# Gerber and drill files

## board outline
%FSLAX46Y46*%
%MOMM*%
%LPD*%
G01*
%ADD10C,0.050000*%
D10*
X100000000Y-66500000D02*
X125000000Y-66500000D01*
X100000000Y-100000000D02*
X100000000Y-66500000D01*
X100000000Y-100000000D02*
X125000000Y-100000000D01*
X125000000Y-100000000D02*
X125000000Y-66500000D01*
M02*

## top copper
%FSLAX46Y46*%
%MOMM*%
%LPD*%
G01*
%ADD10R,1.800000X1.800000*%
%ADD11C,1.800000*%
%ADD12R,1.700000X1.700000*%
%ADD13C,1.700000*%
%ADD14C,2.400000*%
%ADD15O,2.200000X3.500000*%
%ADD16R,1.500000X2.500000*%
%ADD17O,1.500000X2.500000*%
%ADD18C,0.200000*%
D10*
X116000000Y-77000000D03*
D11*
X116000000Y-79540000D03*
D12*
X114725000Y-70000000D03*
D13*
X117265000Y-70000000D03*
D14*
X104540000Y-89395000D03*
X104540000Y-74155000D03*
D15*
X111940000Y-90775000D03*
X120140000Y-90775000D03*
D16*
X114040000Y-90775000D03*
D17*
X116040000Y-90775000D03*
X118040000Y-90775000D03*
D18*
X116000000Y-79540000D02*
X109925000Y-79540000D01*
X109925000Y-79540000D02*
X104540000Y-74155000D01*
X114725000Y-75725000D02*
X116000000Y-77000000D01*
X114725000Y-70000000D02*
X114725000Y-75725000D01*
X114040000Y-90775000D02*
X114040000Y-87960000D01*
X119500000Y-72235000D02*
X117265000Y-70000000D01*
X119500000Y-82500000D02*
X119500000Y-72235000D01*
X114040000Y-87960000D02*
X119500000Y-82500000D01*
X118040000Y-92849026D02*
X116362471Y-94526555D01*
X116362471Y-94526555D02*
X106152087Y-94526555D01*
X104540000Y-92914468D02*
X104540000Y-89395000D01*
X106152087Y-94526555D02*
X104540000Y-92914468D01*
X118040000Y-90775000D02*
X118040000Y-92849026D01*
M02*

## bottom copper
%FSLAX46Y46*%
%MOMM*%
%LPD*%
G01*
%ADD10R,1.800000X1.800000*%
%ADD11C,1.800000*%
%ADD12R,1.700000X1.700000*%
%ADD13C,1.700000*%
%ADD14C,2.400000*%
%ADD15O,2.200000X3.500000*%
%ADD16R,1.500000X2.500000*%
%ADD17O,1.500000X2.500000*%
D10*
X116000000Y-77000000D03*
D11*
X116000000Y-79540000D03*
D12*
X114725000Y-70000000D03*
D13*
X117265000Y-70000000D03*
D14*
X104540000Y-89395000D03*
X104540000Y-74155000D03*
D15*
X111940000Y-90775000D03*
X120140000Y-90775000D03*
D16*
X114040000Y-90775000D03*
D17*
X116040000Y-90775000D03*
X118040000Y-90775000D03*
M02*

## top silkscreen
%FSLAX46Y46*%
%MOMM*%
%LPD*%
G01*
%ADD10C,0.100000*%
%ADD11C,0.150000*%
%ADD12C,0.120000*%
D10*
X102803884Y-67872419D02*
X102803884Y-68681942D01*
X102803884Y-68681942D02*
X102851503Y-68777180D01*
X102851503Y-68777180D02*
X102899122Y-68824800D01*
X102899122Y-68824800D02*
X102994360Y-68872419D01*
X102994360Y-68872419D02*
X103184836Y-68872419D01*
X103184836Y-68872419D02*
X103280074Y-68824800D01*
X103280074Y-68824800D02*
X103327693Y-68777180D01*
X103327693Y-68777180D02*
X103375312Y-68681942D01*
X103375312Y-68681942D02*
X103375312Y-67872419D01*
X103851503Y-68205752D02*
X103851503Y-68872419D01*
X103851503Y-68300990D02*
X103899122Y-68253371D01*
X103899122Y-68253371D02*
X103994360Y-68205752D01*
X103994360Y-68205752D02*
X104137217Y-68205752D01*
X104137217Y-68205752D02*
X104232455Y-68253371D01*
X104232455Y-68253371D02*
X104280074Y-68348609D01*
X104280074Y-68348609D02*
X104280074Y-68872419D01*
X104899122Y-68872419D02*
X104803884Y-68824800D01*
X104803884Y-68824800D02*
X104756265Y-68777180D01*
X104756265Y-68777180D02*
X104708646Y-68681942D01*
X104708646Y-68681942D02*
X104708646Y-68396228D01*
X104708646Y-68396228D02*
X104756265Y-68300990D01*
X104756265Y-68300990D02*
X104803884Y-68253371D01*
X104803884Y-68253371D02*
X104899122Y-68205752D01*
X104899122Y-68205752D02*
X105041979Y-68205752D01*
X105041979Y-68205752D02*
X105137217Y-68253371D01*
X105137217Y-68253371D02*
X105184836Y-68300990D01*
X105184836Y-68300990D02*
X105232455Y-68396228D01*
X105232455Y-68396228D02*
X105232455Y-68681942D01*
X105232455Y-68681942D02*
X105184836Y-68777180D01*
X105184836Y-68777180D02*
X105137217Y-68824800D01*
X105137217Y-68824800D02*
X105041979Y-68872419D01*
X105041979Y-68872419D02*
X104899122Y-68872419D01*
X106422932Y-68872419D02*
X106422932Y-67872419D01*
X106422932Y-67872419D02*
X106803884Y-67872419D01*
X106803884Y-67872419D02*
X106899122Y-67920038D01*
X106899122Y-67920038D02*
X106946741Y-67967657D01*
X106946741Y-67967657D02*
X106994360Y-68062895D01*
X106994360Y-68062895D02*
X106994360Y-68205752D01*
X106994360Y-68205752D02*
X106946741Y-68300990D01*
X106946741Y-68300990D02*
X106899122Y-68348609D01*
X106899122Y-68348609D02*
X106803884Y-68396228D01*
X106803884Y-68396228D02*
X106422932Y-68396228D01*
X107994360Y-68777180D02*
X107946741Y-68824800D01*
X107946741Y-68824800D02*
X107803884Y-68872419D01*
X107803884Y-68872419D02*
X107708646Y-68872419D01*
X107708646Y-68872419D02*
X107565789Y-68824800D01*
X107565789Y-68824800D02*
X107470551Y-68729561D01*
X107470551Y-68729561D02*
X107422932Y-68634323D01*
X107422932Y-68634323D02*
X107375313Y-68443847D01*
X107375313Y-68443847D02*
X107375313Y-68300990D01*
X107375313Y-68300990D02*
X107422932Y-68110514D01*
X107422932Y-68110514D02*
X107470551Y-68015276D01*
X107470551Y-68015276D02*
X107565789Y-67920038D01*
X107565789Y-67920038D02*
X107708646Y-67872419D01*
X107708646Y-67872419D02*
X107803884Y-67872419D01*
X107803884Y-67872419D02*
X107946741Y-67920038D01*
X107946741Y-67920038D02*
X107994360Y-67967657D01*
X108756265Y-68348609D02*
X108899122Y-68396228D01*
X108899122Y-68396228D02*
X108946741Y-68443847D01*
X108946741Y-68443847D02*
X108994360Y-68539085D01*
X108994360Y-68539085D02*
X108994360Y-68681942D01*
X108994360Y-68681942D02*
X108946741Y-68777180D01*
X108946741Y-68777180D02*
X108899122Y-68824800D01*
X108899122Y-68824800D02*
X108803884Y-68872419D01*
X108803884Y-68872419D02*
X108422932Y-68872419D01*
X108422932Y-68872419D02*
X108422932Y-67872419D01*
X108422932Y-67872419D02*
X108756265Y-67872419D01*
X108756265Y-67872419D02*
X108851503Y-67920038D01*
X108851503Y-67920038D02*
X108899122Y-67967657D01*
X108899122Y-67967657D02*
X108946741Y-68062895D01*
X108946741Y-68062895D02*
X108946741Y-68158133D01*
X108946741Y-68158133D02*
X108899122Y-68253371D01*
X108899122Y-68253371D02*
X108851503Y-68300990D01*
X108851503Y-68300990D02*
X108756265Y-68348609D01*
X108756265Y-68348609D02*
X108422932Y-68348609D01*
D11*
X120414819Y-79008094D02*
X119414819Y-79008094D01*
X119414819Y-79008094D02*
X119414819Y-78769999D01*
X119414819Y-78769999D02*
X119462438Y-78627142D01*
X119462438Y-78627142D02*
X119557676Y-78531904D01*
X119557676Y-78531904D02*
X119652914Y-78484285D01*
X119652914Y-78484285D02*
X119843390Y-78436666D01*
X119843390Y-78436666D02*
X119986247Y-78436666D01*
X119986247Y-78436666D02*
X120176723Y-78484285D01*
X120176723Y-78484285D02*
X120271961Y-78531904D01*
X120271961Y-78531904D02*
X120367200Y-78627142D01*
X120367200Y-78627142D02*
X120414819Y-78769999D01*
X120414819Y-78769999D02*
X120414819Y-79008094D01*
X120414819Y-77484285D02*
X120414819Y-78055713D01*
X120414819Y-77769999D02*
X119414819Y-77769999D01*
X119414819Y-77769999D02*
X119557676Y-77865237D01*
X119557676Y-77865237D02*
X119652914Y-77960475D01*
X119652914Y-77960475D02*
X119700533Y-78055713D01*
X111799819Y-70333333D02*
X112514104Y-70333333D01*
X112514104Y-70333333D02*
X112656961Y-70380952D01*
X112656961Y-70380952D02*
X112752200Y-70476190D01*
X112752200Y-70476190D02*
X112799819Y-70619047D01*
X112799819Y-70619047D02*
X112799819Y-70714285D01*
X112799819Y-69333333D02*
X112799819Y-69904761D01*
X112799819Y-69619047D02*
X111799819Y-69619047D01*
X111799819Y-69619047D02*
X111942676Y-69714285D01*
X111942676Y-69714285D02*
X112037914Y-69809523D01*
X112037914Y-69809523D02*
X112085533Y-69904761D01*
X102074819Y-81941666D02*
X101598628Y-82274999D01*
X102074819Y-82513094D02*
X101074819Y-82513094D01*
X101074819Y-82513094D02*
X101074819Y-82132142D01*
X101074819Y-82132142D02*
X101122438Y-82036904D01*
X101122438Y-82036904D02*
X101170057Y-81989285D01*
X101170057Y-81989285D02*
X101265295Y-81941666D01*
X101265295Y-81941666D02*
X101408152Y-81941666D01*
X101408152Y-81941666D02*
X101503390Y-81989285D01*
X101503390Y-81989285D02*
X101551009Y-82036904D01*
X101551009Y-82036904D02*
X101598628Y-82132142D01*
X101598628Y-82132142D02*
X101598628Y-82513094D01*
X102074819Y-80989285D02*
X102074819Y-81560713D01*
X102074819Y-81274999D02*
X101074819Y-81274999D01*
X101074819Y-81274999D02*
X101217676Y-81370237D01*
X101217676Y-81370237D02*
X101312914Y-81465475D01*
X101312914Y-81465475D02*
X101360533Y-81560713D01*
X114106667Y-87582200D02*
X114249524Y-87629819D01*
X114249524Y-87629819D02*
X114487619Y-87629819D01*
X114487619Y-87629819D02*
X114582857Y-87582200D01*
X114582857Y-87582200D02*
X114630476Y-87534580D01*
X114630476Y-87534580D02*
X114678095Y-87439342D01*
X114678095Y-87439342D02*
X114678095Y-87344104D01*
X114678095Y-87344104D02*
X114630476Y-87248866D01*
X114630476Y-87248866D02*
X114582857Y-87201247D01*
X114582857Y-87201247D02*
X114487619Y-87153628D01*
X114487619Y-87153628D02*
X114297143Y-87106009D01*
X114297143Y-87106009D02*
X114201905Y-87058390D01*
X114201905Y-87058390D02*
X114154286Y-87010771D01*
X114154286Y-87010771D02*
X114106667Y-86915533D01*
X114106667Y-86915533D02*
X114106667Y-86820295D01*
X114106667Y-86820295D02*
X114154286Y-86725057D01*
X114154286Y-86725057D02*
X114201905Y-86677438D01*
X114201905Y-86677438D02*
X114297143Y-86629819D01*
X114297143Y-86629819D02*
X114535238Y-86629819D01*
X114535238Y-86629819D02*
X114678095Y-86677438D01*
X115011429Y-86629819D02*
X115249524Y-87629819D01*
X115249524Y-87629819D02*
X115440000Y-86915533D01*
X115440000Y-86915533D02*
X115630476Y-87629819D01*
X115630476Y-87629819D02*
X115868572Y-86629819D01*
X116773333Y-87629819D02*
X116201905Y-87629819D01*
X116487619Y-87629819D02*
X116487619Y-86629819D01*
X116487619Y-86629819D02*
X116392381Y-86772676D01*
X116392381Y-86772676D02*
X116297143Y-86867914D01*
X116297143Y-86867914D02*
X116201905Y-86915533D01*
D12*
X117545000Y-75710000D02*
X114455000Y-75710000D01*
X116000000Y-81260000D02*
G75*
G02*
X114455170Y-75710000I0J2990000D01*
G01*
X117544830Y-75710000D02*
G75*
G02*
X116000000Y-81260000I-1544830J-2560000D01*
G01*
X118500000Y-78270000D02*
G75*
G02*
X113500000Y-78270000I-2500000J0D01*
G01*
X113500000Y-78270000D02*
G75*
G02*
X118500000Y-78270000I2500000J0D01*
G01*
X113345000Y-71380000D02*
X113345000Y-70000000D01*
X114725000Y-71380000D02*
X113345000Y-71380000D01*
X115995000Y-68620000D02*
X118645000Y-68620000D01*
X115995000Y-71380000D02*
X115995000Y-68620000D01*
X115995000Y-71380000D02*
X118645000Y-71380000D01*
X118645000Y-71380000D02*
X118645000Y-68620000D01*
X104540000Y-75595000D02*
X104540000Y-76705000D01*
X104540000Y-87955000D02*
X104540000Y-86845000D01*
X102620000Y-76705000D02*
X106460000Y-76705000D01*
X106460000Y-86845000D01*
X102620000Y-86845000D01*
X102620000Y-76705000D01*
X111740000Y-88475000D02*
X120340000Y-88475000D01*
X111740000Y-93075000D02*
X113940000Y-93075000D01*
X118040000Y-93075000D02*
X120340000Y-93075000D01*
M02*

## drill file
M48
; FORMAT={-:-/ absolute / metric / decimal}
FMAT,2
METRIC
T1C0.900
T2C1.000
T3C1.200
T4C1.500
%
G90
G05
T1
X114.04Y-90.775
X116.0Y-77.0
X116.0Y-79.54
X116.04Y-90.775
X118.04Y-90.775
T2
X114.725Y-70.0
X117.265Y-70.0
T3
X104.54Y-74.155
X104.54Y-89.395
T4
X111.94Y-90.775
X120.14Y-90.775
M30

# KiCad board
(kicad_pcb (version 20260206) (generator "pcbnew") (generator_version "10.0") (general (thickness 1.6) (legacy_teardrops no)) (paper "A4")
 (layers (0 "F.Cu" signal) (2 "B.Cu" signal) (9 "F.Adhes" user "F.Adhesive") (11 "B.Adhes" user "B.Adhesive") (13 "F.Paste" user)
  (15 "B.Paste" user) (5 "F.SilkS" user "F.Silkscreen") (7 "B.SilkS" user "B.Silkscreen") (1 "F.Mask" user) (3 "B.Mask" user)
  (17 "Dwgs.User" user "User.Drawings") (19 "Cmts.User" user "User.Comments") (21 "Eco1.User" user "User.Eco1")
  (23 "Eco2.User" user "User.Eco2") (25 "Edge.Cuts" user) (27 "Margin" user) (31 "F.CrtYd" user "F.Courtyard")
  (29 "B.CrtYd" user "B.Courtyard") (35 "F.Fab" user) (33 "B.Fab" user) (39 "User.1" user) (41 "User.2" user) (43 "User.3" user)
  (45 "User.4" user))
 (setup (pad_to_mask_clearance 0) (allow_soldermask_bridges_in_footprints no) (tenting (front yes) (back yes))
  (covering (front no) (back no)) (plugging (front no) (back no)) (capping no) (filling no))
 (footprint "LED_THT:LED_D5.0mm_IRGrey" (layer "F.Cu") (at 116 77 -90)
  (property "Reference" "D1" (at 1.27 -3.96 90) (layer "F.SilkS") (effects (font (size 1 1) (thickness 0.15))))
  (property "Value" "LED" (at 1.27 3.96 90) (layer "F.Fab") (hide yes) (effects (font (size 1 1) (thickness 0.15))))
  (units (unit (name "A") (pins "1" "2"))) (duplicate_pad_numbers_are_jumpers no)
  (fp_line (start -1.29 -1.545) (end -1.29 1.545) (stroke (width 0.12) (type solid)) (layer "F.SilkS"))
  (fp_arc (start 4.26 0) (mid 2.071779 2.880495) (end -1.29 1.54483) (stroke (width 0.12) (type solid)) (layer "F.SilkS"))
  (fp_arc (start -1.29 -1.54483) (mid 2.071779 -2.880495) (end 4.26 0) (stroke (width 0.12) (type solid)) (layer "F.SilkS"))
  (fp_circle (center 1.27 0) (end 3.77 0) (stroke (width 0.12) (type solid)) (fill no) (layer "F.SilkS"))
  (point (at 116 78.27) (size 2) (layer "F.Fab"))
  (pad "1" thru_hole rect (at 0 0 270) (size 1.8 1.8) (drill 0.9) (layers "*.Cu" "*.Mask") (remove_unused_layers no) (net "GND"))
  (pad "2" thru_hole circle (at 2.54 0 270) (size 1.8 1.8) (drill 0.9) (layers "*.Cu" "*.Mask") (remove_unused_layers no) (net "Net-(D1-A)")))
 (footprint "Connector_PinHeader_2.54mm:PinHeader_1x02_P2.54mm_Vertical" (layer "F.Cu") (at 114.725 70 90)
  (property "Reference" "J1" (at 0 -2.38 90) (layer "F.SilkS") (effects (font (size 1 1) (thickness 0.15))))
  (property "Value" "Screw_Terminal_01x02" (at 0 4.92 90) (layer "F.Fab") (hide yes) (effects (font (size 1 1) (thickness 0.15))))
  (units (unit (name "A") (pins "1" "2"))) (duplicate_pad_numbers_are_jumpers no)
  (fp_line (start -1.38 -1.38) (end 0 -1.38) (stroke (width 0.12) (type solid)) (layer "F.SilkS"))
  (fp_line (start -1.38 0) (end -1.38 -1.38) (stroke (width 0.12) (type solid)) (layer "F.SilkS"))
  (fp_line (start 1.38 1.27) (end 1.38 3.92) (stroke (width 0.12) (type solid)) (layer "F.SilkS"))
  (fp_line (start -1.38 1.27) (end 1.38 1.27) (stroke (width 0.12) (type solid)) (layer "F.SilkS"))
  (fp_line (start -1.38 1.27) (end -1.38 3.92) (stroke (width 0.12) (type solid)) (layer "F.SilkS"))
  (fp_line (start -1.38 3.92) (end 1.38 3.92) (stroke (width 0.12) (type solid)) (layer "F.SilkS"))
  (pad "1" thru_hole rect (at 0 0 90) (size 1.7 1.7) (drill 1) (layers "*.Cu" "*.Mask") (remove_unused_layers no) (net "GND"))
  (pad "2" thru_hole circle (at 0 2.54 90) (size 1.7 1.7) (drill 1) (layers "*.Cu" "*.Mask") (remove_unused_layers no) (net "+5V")))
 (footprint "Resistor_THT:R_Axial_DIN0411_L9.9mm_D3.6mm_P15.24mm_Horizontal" (layer "F.Cu") (at 104.54 89.395 90)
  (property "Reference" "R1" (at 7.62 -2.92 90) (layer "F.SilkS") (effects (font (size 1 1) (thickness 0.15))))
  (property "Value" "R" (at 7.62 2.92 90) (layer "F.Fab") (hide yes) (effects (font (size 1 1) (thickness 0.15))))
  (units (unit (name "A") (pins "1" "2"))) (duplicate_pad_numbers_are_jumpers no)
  (fp_line (start 13.8 0) (end 12.69 0) (stroke (width 0.12) (type solid)) (layer "F.SilkS"))
  (fp_line (start 1.44 0) (end 2.55 0) (stroke (width 0.12) (type solid)) (layer "F.SilkS"))
  (fp_rect (start 2.55 -1.92) (end 12.69 1.92) (stroke (width 0.12) (type solid)) (fill no) (layer "F.SilkS"))
  (pad "1" thru_hole circle (at 0 0 90) (size 2.4 2.4) (drill 1.2) (layers "*.Cu" "*.Mask") (remove_unused_layers no) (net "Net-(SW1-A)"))
  (pad "2" thru_hole circle (at 15.24 0 90) (size 2.4 2.4) (drill 1.2) (layers "*.Cu" "*.Mask") (remove_unused_layers no) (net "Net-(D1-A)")))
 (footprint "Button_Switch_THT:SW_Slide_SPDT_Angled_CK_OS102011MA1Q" (layer "F.Cu") (at 114.04 90.775)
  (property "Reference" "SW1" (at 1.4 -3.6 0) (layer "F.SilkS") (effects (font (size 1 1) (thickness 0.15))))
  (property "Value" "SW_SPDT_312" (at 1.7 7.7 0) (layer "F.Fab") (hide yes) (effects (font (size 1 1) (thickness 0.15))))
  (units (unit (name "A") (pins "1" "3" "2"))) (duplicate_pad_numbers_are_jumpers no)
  (fp_line (start -2.3 -2.3) (end 6.3 -2.3) (stroke (width 0.12) (type solid)) (layer "F.SilkS"))
  (fp_line (start -2.3 2.3) (end -0.1 2.3) (stroke (width 0.12) (type solid)) (layer "F.SilkS"))
  (fp_line (start 4 2.3) (end 6.3 2.3) (stroke (width 0.12) (type solid)) (layer "F.SilkS"))
  (pad "" thru_hole oval (at -2.1 0) (size 2.2 3.5) (drill 1.5) (layers "*.Cu" "*.Mask") (remove_unused_layers no))
  (pad "" thru_hole oval (at 6.1 0) (size 2.2 3.5) (drill 1.5) (layers "*.Cu" "*.Mask") (remove_unused_layers no))
  (pad "1" thru_hole rect (at 0 0) (size 1.5 2.5) (drill 0.9) (layers "*.Cu" "*.Mask") (remove_unused_layers no) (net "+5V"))
  (pad "2" thru_hole oval (at 2 0) (size 1.5 2.5) (drill 0.9) (layers "*.Cu" "*.Mask") (remove_unused_layers no)
   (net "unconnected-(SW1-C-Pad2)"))
  (pad "3" thru_hole oval (at 4 0) (size 1.5 2.5) (drill 0.9) (layers "*.Cu" "*.Mask") (remove_unused_layers no) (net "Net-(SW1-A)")))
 (gr_line (start 100 66.5) (end 125 66.5) (stroke (width 0.05) (type solid)) (layer "Edge.Cuts"))
 (gr_line (start 100 100) (end 100 66.5) (stroke (width 0.05) (type solid)) (layer "Edge.Cuts"))
 (gr_line (start 100 100) (end 125 100) (stroke (width 0.05) (type solid)) (layer "Edge.Cuts"))
 (gr_line (start 125 100) (end 125 66.5) (stroke (width 0.05) (type solid)) (layer "Edge.Cuts"))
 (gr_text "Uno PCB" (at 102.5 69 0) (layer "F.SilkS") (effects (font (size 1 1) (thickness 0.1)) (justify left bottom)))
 (segment (start 116 79.54) (end 109.925 79.54) (width 0.2) (layer "F.Cu") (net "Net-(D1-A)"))
 (segment (start 109.925 79.54) (end 104.54 74.155) (width 0.2) (layer "F.Cu") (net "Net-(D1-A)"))
 (segment (start 114.725 75.725) (end 116 77) (width 0.2) (layer "F.Cu") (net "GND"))
 (segment (start 114.725 70) (end 114.725 75.725) (width 0.2) (layer "F.Cu") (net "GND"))
 (segment (start 114.04 90.775) (end 114.04 87.96) (width 0.2) (layer "F.Cu") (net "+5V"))
 (segment (start 119.5 72.235) (end 117.265 70) (width 0.2) (layer "F.Cu") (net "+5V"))
 (segment (start 119.5 82.5) (end 119.5 72.235) (width 0.2) (layer "F.Cu") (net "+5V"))
 (segment (start 114.04 87.96) (end 119.5 82.5) (width 0.2) (layer "F.Cu") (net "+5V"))
 (segment (start 118.04 92.849026) (end 116.362471 94.526555) (width 0.2) (layer "F.Cu") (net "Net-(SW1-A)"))
 (segment (start 116.362471 94.526555) (end 106.152087 94.526555) (width 0.2) (layer "F.Cu") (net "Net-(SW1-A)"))
 (segment (start 104.54 92.914468) (end 104.54 89.395) (width 0.2) (layer "F.Cu") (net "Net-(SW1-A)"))
 (segment (start 106.152087 94.526555) (end 104.54 92.914468) (width 0.2) (layer "F.Cu") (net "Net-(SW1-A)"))
 (segment (start 118.04 90.775) (end 118.04 92.849026) (width 0.2) (layer "F.Cu") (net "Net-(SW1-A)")))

